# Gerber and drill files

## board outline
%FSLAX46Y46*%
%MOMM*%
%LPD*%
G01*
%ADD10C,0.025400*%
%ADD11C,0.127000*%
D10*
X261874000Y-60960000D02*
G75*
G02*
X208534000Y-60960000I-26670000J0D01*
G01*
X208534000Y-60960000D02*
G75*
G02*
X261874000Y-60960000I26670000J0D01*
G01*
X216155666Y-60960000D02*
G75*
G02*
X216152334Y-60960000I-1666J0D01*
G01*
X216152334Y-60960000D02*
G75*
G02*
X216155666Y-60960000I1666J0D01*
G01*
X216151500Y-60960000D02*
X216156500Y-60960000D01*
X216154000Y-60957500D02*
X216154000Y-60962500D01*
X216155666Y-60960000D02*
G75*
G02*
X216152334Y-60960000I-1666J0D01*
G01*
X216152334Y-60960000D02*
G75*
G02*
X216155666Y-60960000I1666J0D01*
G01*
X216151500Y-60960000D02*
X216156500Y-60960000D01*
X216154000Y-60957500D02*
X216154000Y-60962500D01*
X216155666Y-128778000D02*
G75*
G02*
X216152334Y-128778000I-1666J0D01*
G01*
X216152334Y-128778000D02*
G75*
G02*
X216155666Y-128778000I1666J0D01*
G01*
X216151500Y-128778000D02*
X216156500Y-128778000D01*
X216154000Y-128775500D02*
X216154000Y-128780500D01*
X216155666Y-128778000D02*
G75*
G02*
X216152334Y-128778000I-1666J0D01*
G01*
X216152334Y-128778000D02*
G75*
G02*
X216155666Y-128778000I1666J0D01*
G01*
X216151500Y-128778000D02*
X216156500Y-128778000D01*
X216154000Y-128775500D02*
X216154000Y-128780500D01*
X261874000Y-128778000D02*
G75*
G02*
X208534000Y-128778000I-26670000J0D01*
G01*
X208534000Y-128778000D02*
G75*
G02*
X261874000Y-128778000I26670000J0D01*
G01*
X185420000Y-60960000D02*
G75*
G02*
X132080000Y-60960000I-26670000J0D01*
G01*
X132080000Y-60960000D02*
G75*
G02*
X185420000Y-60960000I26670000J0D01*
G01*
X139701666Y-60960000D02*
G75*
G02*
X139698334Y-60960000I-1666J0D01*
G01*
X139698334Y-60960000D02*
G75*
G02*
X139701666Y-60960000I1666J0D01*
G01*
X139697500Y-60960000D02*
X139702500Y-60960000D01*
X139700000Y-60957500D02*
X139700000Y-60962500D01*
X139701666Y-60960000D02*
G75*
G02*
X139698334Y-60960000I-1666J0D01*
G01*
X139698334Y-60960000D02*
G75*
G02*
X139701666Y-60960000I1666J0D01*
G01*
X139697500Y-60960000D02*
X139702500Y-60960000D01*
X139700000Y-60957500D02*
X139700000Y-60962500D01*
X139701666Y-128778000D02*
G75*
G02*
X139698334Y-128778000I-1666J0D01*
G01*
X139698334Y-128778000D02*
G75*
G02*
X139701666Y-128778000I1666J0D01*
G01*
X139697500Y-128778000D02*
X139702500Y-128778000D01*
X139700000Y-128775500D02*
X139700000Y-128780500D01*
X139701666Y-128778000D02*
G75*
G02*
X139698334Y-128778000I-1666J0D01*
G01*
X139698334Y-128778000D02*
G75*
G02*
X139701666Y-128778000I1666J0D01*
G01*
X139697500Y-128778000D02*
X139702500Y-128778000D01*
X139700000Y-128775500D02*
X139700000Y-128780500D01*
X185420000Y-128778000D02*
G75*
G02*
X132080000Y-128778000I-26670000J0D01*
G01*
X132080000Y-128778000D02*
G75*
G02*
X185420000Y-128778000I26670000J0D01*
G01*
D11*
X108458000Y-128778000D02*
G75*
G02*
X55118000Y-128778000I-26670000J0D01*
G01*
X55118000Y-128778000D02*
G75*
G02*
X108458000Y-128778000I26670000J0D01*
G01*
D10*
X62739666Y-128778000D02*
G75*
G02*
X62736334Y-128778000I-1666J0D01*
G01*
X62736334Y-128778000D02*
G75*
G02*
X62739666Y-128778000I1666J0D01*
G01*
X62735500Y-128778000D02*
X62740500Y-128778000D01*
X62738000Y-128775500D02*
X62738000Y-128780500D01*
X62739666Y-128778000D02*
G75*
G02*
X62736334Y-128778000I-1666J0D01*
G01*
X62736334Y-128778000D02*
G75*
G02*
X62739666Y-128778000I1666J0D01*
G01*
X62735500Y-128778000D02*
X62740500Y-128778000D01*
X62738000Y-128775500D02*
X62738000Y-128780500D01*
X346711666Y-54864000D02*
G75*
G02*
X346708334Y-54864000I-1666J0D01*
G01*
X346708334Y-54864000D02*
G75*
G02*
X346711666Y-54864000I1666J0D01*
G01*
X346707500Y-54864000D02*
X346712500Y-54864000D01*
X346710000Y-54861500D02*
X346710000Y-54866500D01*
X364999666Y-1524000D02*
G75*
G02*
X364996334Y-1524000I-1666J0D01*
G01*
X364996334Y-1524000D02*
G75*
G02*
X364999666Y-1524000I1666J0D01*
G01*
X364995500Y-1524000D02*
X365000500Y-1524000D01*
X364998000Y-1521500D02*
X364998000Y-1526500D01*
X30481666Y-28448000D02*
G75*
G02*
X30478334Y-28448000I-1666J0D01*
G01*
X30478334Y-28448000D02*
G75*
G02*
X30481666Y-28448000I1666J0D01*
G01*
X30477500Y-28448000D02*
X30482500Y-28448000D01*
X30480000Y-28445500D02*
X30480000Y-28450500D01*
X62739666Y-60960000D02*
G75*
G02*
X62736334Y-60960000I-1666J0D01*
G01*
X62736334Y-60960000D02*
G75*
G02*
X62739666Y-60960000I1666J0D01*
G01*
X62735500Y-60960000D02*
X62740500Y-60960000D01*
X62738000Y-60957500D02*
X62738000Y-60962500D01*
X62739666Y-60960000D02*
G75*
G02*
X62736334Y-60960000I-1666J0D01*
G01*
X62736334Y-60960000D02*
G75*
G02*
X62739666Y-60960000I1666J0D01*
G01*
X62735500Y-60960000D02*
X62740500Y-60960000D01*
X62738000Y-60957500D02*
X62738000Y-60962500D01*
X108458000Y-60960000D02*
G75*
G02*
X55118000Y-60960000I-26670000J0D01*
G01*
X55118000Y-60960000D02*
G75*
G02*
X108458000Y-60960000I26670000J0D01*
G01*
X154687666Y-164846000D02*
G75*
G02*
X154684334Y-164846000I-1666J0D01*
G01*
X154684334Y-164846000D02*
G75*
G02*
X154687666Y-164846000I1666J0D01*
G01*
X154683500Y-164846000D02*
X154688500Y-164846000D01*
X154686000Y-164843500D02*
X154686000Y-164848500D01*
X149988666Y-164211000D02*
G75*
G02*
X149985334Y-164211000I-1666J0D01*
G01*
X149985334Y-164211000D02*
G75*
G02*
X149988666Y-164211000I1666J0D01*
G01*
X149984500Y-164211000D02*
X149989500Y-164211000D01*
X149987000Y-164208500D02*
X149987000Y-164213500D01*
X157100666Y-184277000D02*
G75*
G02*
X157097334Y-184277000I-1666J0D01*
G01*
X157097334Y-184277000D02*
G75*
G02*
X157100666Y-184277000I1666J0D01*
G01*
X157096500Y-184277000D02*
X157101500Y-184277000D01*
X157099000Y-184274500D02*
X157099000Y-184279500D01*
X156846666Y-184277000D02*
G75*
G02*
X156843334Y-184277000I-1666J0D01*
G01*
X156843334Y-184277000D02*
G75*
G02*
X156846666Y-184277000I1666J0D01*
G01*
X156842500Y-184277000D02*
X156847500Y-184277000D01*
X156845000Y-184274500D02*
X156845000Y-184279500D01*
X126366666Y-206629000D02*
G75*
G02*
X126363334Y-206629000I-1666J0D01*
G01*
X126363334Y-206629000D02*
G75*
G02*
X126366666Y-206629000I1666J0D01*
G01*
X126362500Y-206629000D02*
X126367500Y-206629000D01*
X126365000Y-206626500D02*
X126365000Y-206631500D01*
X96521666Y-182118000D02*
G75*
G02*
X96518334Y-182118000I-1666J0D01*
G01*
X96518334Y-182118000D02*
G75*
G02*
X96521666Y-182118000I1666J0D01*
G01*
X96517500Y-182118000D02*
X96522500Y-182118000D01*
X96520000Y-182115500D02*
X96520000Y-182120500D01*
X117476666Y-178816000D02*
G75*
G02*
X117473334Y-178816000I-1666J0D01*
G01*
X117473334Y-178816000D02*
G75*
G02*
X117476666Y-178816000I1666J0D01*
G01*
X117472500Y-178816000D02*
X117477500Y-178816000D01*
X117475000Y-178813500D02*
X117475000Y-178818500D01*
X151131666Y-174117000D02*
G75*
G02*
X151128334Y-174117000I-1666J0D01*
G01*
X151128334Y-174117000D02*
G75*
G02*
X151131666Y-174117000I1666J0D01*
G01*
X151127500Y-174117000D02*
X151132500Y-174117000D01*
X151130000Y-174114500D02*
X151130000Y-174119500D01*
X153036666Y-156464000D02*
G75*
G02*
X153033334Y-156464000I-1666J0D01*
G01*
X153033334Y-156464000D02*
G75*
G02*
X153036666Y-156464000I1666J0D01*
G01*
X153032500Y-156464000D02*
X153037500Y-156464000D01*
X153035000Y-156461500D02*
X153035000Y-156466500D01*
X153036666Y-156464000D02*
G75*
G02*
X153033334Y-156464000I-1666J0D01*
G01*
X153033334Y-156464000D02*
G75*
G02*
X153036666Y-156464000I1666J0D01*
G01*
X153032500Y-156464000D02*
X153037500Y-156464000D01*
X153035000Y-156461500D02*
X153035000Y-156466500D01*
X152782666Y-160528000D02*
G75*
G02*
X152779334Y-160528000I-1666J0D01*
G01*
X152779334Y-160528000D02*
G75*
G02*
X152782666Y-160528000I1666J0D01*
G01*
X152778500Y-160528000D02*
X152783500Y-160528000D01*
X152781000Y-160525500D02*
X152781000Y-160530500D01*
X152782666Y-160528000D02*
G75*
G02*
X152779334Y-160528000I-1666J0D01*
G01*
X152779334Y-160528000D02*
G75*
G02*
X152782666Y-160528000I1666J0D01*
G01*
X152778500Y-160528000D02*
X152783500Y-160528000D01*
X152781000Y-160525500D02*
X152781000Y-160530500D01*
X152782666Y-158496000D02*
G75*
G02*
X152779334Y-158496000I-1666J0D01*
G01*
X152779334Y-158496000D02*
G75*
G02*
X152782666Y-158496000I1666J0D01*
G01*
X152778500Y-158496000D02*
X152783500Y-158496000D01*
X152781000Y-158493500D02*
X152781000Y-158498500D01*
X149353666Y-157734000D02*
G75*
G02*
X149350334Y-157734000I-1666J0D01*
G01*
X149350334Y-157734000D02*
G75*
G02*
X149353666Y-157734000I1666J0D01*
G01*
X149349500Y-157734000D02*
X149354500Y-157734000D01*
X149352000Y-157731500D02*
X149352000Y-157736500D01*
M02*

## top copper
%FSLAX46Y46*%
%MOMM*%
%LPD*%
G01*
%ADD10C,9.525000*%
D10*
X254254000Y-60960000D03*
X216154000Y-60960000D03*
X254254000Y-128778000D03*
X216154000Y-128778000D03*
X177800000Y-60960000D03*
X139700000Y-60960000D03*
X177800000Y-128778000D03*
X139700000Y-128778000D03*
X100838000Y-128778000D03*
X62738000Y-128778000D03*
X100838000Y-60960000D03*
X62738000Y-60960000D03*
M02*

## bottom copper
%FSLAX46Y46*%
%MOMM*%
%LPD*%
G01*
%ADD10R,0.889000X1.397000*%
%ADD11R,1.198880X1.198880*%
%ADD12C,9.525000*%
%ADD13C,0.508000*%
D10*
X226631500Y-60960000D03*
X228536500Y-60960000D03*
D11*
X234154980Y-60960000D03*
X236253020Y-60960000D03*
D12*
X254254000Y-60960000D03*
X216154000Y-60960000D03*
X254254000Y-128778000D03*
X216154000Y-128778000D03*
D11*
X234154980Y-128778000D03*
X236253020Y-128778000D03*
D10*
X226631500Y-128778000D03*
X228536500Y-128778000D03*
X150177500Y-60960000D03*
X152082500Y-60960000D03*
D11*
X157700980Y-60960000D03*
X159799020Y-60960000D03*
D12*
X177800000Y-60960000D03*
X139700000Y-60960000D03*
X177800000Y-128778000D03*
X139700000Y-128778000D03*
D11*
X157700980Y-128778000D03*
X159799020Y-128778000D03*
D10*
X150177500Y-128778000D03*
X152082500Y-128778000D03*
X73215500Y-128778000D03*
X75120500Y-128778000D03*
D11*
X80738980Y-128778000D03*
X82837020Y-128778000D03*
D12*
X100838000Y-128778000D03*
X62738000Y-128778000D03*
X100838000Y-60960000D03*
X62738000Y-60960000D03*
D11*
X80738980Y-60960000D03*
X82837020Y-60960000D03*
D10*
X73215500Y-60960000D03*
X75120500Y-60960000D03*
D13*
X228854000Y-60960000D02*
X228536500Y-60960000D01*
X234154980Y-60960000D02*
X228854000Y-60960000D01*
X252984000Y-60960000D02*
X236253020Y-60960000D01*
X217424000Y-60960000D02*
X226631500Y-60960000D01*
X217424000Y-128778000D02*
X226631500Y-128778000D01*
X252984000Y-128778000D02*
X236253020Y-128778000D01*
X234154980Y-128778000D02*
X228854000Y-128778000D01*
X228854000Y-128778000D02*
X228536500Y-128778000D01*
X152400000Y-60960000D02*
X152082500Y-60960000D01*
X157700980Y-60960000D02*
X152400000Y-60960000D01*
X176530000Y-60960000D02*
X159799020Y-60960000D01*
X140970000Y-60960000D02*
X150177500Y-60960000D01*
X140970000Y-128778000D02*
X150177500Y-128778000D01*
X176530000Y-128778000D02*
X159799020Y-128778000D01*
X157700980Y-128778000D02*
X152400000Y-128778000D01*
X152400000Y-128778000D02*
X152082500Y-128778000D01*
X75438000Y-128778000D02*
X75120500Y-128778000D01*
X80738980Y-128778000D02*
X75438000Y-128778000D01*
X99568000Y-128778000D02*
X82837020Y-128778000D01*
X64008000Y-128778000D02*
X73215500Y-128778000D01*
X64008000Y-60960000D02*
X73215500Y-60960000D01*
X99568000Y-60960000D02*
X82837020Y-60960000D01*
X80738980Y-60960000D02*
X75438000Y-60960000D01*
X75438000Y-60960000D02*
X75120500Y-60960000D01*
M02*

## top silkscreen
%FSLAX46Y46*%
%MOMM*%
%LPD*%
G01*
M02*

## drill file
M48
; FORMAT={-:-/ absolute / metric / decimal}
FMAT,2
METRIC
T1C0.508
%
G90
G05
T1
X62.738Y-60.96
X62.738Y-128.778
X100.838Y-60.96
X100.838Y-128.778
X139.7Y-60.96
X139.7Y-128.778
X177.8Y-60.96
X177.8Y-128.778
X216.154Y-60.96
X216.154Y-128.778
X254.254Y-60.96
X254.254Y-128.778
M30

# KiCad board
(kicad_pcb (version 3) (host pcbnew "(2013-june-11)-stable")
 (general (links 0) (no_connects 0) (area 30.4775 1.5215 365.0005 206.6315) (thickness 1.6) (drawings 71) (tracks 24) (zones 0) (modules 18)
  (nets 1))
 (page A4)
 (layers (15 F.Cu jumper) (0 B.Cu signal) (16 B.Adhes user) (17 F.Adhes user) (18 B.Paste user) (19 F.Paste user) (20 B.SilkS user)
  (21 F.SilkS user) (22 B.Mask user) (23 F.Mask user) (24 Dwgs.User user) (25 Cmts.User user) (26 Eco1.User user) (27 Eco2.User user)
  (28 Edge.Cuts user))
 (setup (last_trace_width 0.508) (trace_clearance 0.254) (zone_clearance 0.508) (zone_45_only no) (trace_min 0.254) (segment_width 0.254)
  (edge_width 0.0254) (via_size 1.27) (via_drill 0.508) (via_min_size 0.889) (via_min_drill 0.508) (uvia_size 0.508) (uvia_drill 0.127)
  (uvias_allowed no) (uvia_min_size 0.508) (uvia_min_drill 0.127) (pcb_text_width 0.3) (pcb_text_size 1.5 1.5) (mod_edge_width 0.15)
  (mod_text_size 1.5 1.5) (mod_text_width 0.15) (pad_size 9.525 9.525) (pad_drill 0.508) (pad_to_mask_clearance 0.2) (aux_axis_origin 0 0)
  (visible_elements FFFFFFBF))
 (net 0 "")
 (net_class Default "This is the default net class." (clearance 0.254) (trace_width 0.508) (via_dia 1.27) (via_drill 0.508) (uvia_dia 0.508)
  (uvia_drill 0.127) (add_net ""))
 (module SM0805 (layer B.Cu) (at 227.584 60.96)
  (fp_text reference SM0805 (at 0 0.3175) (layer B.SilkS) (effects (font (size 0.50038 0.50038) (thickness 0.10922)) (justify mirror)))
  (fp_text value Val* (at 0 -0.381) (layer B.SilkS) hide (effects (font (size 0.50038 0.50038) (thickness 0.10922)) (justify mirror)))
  (pad 1 smd rect (at -0.9525 0) (size 0.889 1.397) (layers B.Cu B.Paste B.Mask))
  (pad 2 smd rect (at 0.9525 0) (size 0.889 1.397) (layers B.Cu B.Paste B.Mask)))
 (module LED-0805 (layer B.Cu) (at 235.204 60.96)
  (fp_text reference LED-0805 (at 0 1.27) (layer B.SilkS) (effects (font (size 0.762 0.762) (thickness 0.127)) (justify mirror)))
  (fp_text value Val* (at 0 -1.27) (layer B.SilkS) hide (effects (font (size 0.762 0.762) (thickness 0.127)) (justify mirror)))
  (pad 1 smd rect (at -1.04902 0) (size 1.19888 1.19888) (layers B.Cu B.Paste B.Mask))
  (pad 2 smd rect (at 1.04902 0) (size 1.19888 1.19888) (layers B.Cu B.Paste B.Mask)))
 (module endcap (layer F.Cu) (at 235.204 60.96)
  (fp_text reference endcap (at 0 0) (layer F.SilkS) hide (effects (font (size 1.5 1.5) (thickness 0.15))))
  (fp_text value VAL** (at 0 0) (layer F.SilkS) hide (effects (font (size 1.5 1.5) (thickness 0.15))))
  (pad "" thru_hole circle (at 19.05 0) (size 9.525 9.525) (drill 0.508) (layers B.Cu) (zone_connect 2))
  (pad "" thru_hole circle (at -19.05 0) (size 9.525 9.525) (drill 0.508) (layers *.Mask B.Cu) (zone_connect 2)))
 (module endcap (layer F.Cu) (at 235.204 128.778)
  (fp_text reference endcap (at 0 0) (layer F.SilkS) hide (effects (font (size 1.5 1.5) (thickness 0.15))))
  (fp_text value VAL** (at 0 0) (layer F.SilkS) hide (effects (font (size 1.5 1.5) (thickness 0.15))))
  (pad "" thru_hole circle (at 19.05 0) (size 9.525 9.525) (drill 0.508) (layers B.Cu) (zone_connect 2))
  (pad "" thru_hole circle (at -19.05 0) (size 9.525 9.525) (drill 0.508) (layers *.Mask B.Cu) (zone_connect 2)))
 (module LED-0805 (layer B.Cu) (at 235.204 128.778)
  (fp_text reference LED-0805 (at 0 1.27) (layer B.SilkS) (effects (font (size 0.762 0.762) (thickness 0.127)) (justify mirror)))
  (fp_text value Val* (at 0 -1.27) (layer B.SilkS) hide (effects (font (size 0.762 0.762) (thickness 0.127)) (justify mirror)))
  (pad 1 smd rect (at -1.04902 0) (size 1.19888 1.19888) (layers B.Cu B.Paste B.Mask))
  (pad 2 smd rect (at 1.04902 0) (size 1.19888 1.19888) (layers B.Cu B.Paste B.Mask)))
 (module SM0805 (layer B.Cu) (at 227.584 128.778)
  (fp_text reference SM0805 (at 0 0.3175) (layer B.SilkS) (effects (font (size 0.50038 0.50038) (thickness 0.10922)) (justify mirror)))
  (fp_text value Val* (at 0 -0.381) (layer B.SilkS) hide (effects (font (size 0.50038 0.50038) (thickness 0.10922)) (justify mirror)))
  (pad 1 smd rect (at -0.9525 0) (size 0.889 1.397) (layers B.Cu B.Paste B.Mask))
  (pad 2 smd rect (at 0.9525 0) (size 0.889 1.397) (layers B.Cu B.Paste B.Mask)))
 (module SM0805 (layer B.Cu) (at 151.13 60.96)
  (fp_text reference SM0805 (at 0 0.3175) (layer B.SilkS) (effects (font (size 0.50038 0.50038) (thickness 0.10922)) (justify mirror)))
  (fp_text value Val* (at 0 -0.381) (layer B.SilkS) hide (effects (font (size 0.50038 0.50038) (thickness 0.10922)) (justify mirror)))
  (pad 1 smd rect (at -0.9525 0) (size 0.889 1.397) (layers B.Cu B.Paste B.Mask))
  (pad 2 smd rect (at 0.9525 0) (size 0.889 1.397) (layers B.Cu B.Paste B.Mask)))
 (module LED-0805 (layer B.Cu) (at 158.75 60.96)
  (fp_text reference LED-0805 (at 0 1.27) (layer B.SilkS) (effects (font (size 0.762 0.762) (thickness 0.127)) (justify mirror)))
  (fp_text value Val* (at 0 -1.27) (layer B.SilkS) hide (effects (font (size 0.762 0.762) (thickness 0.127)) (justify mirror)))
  (pad 1 smd rect (at -1.04902 0) (size 1.19888 1.19888) (layers B.Cu B.Paste B.Mask))
  (pad 2 smd rect (at 1.04902 0) (size 1.19888 1.19888) (layers B.Cu B.Paste B.Mask)))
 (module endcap (layer F.Cu) (at 158.75 60.96)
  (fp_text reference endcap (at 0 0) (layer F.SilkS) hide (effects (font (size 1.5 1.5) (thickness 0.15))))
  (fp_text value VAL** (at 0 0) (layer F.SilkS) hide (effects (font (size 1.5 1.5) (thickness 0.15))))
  (pad "" thru_hole circle (at 19.05 0) (size 9.525 9.525) (drill 0.508) (layers B.Cu) (zone_connect 2))
  (pad "" thru_hole circle (at -19.05 0) (size 9.525 9.525) (drill 0.508) (layers *.Mask B.Cu) (zone_connect 2)))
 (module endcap (layer F.Cu) (at 158.75 128.778)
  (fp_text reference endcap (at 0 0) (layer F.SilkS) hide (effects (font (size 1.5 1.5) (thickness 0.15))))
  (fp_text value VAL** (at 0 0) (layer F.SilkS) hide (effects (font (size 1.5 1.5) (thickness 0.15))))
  (pad "" thru_hole circle (at 19.05 0) (size 9.525 9.525) (drill 0.508) (layers B.Cu) (zone_connect 2))
  (pad "" thru_hole circle (at -19.05 0) (size 9.525 9.525) (drill 0.508) (layers *.Mask B.Cu) (zone_connect 2)))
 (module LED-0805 (layer B.Cu) (at 158.75 128.778)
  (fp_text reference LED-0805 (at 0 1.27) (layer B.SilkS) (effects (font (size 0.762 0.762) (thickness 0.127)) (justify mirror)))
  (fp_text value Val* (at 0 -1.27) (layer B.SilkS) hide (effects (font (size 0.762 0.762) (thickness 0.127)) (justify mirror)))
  (pad 1 smd rect (at -1.04902 0) (size 1.19888 1.19888) (layers B.Cu B.Paste B.Mask))
  (pad 2 smd rect (at 1.04902 0) (size 1.19888 1.19888) (layers B.Cu B.Paste B.Mask)))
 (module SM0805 (layer B.Cu) (at 151.13 128.778)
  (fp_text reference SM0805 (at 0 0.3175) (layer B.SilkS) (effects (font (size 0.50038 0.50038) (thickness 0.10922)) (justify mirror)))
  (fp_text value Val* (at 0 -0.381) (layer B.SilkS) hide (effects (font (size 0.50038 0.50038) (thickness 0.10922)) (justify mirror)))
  (pad 1 smd rect (at -0.9525 0) (size 0.889 1.397) (layers B.Cu B.Paste B.Mask))
  (pad 2 smd rect (at 0.9525 0) (size 0.889 1.397) (layers B.Cu B.Paste B.Mask)))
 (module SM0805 (layer B.Cu) (at 74.168 128.778)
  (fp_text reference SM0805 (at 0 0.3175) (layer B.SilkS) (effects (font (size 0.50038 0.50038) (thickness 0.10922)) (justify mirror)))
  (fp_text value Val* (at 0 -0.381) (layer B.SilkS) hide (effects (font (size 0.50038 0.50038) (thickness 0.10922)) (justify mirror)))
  (pad 1 smd rect (at -0.9525 0) (size 0.889 1.397) (layers B.Cu B.Paste B.Mask))
  (pad 2 smd rect (at 0.9525 0) (size 0.889 1.397) (layers B.Cu B.Paste B.Mask)))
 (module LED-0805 (layer B.Cu) (at 81.788 128.778)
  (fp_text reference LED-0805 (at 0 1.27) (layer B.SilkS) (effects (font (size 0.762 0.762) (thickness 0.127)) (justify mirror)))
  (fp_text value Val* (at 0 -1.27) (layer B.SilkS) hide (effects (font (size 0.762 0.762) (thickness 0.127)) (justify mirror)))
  (pad 1 smd rect (at -1.04902 0) (size 1.19888 1.19888) (layers B.Cu B.Paste B.Mask))
  (pad 2 smd rect (at 1.04902 0) (size 1.19888 1.19888) (layers B.Cu B.Paste B.Mask)))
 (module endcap (layer F.Cu) (at 81.788 128.778)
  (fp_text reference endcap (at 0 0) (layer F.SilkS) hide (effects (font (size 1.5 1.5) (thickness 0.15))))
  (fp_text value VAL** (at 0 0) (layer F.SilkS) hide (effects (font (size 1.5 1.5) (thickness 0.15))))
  (pad "" thru_hole circle (at 19.05 0) (size 9.525 9.525) (drill 0.508) (layers B.Cu) (zone_connect 2))
  (pad "" thru_hole circle (at -19.05 0) (size 9.525 9.525) (drill 0.508) (layers *.Mask B.Cu) (zone_connect 2)))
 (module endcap (layer F.Cu) (at 81.788 60.96)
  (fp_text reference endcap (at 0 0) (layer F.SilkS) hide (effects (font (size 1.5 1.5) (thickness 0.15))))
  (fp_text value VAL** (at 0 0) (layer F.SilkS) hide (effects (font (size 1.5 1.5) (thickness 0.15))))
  (pad "" thru_hole circle (at 19.05 0) (size 9.525 9.525) (drill 0.508) (layers B.Cu) (zone_connect 2))
  (pad "" thru_hole circle (at -19.05 0) (size 9.525 9.525) (drill 0.508) (layers *.Mask B.Cu) (zone_connect 2)))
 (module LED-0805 (layer B.Cu) (at 81.788 60.96)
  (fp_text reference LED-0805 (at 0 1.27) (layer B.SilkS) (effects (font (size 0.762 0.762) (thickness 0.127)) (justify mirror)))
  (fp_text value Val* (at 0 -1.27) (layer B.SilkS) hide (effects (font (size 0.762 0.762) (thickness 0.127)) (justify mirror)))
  (pad 1 smd rect (at -1.04902 0) (size 1.19888 1.19888) (layers B.Cu B.Paste B.Mask))
  (pad 2 smd rect (at 1.04902 0) (size 1.19888 1.19888) (layers B.Cu B.Paste B.Mask)))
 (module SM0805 (layer B.Cu) (at 74.168 60.96)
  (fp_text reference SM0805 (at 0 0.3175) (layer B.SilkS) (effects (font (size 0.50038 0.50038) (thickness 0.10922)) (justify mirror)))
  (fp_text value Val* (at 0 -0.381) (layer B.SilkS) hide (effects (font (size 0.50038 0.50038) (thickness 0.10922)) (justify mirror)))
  (pad 1 smd rect (at -0.9525 0) (size 0.889 1.397) (layers B.Cu B.Paste B.Mask))
  (pad 2 smd rect (at 0.9525 0) (size 0.889 1.397) (layers B.Cu B.Paste B.Mask)))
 (gr_circle (center 235.204 60.96) (end 261.874 60.96) (layer Edge.Cuts) (width 0.0254))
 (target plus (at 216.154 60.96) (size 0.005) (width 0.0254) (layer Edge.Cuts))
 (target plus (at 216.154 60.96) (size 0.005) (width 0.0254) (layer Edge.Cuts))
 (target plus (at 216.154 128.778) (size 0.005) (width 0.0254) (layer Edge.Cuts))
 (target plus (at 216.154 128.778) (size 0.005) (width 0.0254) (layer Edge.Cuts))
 (gr_circle (center 235.204 128.778) (end 261.874 128.778) (layer Edge.Cuts) (width 0.0254))
 (gr_circle (center 158.75 60.96) (end 185.42 60.96) (layer Edge.Cuts) (width 0.0254))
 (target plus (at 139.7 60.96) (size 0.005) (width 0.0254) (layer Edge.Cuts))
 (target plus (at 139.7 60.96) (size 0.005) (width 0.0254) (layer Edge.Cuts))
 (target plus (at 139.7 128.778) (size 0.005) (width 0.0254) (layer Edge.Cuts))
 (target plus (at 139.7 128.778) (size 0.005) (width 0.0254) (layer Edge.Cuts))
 (gr_circle (center 158.75 128.778) (end 185.42 128.778) (layer Edge.Cuts) (width 0.0254))
 (gr_circle (center 81.788 128.778) (end 108.458 128.778) (layer Edge.Cuts) (width 0.127))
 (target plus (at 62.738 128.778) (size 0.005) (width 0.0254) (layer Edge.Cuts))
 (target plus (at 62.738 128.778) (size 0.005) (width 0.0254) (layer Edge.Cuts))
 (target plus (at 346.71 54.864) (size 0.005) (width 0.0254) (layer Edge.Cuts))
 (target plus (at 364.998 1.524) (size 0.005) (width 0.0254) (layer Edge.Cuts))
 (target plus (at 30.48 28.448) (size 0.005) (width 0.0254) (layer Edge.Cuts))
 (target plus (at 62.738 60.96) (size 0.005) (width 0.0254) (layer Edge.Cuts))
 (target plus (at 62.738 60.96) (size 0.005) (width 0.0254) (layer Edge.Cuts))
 (gr_circle (center 81.788 60.96) (end 108.458 60.96) (layer Edge.Cuts) (width 0.0254))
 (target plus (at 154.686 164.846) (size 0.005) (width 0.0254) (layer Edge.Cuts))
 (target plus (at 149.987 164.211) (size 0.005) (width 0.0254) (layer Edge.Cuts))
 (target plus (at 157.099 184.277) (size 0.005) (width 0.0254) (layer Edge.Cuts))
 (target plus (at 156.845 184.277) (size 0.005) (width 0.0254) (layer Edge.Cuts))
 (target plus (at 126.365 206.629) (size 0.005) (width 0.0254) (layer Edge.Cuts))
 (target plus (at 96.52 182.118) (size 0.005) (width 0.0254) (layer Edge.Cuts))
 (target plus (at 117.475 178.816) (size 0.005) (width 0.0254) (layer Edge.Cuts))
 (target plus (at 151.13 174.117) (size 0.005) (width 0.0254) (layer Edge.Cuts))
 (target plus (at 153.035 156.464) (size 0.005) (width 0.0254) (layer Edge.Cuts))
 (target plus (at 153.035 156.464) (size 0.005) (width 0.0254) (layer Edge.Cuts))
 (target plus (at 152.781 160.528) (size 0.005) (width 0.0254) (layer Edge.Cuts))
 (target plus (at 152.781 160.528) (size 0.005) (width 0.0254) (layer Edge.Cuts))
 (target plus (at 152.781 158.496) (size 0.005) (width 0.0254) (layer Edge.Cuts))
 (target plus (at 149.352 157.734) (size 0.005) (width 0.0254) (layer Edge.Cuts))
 (segment (start 228.854 60.96) (end 228.5365 60.96) (width 0.508) (layer B.Cu) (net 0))
 (segment (start 234.15498 60.96) (end 228.854 60.96) (width 0.508) (layer B.Cu) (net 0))
 (segment (start 252.984 60.96) (end 236.25302 60.96) (width 0.508) (layer B.Cu) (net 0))
 (segment (start 217.424 60.96) (end 226.6315 60.96) (width 0.508) (layer B.Cu) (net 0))
 (segment (start 217.424 128.778) (end 226.6315 128.778) (width 0.508) (layer B.Cu) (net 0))
 (segment (start 252.984 128.778) (end 236.25302 128.778) (width 0.508) (layer B.Cu) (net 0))
 (segment (start 234.15498 128.778) (end 228.854 128.778) (width 0.508) (layer B.Cu) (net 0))
 (segment (start 228.854 128.778) (end 228.5365 128.778) (width 0.508) (layer B.Cu) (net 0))
 (segment (start 152.4 60.96) (end 152.0825 60.96) (width 0.508) (layer B.Cu) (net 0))
 (segment (start 157.70098 60.96) (end 152.4 60.96) (width 0.508) (layer B.Cu) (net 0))
 (segment (start 176.53 60.96) (end 159.79902 60.96) (width 0.508) (layer B.Cu) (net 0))
 (segment (start 140.97 60.96) (end 150.1775 60.96) (width 0.508) (layer B.Cu) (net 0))
 (segment (start 140.97 128.778) (end 150.1775 128.778) (width 0.508) (layer B.Cu) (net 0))
 (segment (start 176.53 128.778) (end 159.79902 128.778) (width 0.508) (layer B.Cu) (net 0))
 (segment (start 157.70098 128.778) (end 152.4 128.778) (width 0.508) (layer B.Cu) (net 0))
 (segment (start 152.4 128.778) (end 152.0825 128.778) (width 0.508) (layer B.Cu) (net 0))
 (segment (start 75.438 128.778) (end 75.1205 128.778) (width 0.508) (layer B.Cu) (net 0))
 (segment (start 80.73898 128.778) (end 75.438 128.778) (width 0.508) (layer B.Cu) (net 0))
 (segment (start 99.568 128.778) (end 82.83702 128.778) (width 0.508) (layer B.Cu) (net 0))
 (segment (start 64.008 128.778) (end 73.2155 128.778) (width 0.508) (layer B.Cu) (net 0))
 (segment (start 64.008 60.96) (end 73.2155 60.96) (width 0.508) (layer B.Cu) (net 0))
 (segment (start 99.568 60.96) (end 82.83702 60.96) (width 0.508) (layer B.Cu) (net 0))
 (segment (start 80.73898 60.96) (end 75.438 60.96) (width 0.508) (layer B.Cu) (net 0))
 (segment (start 75.438 60.96) (end 75.1205 60.96) (width 0.508) (layer B.Cu) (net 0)))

